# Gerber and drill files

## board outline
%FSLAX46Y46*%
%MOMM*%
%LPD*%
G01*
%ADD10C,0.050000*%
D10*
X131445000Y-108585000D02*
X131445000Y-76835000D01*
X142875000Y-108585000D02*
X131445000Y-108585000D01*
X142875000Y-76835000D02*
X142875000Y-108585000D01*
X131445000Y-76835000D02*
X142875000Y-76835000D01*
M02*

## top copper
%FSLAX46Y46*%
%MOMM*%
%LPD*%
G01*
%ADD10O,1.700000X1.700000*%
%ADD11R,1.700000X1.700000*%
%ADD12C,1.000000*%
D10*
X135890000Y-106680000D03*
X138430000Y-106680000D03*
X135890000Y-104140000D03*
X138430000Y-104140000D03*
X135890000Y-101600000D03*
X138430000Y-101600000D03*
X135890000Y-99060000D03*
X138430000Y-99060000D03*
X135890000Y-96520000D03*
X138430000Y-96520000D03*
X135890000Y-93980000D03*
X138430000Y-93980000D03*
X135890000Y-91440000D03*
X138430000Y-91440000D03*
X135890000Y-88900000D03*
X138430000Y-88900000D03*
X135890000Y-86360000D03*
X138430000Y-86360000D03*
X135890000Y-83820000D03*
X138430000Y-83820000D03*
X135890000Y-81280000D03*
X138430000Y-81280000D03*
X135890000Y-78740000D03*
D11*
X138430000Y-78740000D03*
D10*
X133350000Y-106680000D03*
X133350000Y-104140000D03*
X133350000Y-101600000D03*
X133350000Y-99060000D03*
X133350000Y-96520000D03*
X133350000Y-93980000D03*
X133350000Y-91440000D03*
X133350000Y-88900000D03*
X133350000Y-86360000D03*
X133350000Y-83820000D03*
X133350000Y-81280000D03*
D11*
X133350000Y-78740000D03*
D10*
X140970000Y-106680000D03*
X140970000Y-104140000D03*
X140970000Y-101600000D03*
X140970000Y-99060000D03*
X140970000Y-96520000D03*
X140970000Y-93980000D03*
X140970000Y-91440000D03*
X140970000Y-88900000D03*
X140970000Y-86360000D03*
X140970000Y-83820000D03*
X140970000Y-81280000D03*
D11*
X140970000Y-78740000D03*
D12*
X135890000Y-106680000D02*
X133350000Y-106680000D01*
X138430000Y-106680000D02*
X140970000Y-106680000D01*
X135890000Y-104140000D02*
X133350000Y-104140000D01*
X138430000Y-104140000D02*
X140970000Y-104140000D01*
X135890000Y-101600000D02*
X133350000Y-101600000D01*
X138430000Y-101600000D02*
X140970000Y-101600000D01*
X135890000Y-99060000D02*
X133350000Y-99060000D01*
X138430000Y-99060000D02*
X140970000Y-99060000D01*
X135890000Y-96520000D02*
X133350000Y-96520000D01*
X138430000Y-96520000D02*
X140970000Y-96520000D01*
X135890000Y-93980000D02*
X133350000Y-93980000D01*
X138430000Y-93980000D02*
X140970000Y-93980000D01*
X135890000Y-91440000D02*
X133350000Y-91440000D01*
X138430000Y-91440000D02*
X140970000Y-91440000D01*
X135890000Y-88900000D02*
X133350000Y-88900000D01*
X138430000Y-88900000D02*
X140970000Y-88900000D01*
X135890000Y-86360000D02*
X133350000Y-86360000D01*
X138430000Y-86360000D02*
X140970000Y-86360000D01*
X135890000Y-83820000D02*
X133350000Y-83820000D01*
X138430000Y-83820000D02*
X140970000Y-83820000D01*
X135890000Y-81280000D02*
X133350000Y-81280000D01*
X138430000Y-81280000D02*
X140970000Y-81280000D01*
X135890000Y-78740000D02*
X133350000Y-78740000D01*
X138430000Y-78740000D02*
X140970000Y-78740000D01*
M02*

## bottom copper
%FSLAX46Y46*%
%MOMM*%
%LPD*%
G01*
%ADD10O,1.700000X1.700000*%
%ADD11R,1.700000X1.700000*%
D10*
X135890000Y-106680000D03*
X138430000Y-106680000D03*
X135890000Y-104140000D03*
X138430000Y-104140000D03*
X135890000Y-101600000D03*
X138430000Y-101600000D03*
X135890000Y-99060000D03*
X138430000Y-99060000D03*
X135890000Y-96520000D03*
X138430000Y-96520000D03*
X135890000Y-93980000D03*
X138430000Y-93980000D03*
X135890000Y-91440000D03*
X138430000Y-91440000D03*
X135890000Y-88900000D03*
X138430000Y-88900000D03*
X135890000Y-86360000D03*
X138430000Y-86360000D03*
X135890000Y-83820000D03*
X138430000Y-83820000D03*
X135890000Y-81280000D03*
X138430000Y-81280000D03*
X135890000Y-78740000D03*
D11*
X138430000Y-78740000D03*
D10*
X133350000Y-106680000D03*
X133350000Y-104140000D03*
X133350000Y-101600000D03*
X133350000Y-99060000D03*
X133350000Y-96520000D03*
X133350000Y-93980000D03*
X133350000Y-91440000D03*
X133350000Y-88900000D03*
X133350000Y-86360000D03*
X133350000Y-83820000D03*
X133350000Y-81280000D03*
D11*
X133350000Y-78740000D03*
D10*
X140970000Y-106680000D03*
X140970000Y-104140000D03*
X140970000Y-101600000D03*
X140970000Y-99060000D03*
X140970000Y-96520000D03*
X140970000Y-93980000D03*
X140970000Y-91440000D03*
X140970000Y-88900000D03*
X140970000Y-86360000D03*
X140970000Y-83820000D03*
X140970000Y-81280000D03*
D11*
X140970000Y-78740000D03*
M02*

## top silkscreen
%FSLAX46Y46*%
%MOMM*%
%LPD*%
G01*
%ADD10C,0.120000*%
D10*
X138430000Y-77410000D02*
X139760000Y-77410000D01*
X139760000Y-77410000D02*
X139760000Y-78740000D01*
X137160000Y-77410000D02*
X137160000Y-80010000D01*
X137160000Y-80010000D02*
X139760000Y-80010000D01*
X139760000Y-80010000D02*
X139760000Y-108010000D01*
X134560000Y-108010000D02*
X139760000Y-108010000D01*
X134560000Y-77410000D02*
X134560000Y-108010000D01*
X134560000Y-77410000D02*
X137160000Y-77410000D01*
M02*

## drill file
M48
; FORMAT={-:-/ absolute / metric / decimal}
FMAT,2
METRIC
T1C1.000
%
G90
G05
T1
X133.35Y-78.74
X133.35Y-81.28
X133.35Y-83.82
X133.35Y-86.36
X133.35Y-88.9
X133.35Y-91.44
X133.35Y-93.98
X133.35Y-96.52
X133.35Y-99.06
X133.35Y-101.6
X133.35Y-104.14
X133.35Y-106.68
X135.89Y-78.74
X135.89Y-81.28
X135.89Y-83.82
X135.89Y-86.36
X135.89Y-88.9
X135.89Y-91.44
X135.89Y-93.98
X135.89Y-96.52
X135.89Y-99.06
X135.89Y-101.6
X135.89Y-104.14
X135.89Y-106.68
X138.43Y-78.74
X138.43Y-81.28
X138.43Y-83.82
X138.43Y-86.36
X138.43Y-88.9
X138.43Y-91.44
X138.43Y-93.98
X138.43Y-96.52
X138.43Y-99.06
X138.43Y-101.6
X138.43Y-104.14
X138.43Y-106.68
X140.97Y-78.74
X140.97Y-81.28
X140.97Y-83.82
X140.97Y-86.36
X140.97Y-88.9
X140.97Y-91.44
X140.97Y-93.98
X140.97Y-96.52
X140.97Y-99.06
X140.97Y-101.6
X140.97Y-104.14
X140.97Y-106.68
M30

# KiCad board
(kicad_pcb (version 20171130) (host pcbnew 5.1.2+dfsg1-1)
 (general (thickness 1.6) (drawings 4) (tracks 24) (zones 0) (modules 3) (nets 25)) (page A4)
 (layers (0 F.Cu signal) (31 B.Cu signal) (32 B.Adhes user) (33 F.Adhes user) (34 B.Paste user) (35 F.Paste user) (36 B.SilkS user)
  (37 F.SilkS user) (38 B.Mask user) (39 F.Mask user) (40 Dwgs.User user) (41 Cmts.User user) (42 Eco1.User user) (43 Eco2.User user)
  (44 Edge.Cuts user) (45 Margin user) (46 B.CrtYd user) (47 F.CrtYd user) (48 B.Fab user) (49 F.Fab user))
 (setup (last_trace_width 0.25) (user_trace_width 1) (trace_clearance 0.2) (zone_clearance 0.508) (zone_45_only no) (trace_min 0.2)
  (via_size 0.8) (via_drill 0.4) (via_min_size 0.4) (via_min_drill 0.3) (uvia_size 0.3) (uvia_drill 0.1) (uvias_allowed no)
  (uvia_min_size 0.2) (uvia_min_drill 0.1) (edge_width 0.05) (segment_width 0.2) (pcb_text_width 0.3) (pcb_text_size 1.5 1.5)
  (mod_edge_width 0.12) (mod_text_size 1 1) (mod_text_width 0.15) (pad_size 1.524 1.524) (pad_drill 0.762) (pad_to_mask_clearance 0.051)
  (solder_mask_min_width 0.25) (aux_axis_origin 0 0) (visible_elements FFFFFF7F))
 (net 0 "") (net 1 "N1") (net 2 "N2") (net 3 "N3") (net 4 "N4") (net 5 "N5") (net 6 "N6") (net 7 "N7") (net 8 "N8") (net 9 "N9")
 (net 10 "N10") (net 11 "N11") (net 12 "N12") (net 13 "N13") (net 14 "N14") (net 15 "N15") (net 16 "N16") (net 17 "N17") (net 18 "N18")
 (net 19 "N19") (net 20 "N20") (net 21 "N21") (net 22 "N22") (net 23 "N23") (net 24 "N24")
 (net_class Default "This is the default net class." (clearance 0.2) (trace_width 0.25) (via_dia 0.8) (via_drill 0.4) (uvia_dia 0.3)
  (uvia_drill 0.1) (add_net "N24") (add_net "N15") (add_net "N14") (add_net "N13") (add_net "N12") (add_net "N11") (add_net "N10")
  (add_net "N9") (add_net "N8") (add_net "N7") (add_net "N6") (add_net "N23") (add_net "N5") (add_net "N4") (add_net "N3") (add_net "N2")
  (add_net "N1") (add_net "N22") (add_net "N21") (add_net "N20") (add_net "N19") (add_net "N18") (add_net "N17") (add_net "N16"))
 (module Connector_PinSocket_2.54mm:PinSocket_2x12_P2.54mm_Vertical (layer F.Cu) (at 138.43 78.74)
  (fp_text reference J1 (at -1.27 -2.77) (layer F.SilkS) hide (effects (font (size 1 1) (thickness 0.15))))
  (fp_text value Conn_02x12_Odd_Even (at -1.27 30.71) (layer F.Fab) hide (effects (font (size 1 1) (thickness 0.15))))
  (fp_line (start 0 -1.33) (end 1.33 -1.33) (layer F.SilkS) (width 0.12))
  (fp_line (start 1.33 -1.33) (end 1.33 0) (layer F.SilkS) (width 0.12))
  (fp_line (start -1.27 -1.33) (end -1.27 1.27) (layer F.SilkS) (width 0.12))
  (fp_line (start -1.27 1.27) (end 1.33 1.27) (layer F.SilkS) (width 0.12))
  (fp_line (start 1.33 1.27) (end 1.33 29.27) (layer F.SilkS) (width 0.12))
  (fp_line (start -3.87 29.27) (end 1.33 29.27) (layer F.SilkS) (width 0.12))
  (fp_line (start -3.87 -1.33) (end -3.87 29.27) (layer F.SilkS) (width 0.12))
  (fp_line (start -3.87 -1.33) (end -1.27 -1.33) (layer F.SilkS) (width 0.12))
  (pad 24 thru_hole oval (at -2.54 27.94) (size 1.7 1.7) (drill 1) (layers *.Cu *.Mask) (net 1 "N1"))
  (pad 23 thru_hole oval (at 0 27.94) (size 1.7 1.7) (drill 1) (layers *.Cu *.Mask) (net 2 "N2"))
  (pad 22 thru_hole oval (at -2.54 25.4) (size 1.7 1.7) (drill 1) (layers *.Cu *.Mask) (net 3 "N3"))
  (pad 21 thru_hole oval (at 0 25.4) (size 1.7 1.7) (drill 1) (layers *.Cu *.Mask) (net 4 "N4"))
  (pad 20 thru_hole oval (at -2.54 22.86) (size 1.7 1.7) (drill 1) (layers *.Cu *.Mask) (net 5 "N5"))
  (pad 19 thru_hole oval (at 0 22.86) (size 1.7 1.7) (drill 1) (layers *.Cu *.Mask) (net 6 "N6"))
  (pad 18 thru_hole oval (at -2.54 20.32) (size 1.7 1.7) (drill 1) (layers *.Cu *.Mask) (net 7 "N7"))
  (pad 17 thru_hole oval (at 0 20.32) (size 1.7 1.7) (drill 1) (layers *.Cu *.Mask) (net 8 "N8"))
  (pad 16 thru_hole oval (at -2.54 17.78) (size 1.7 1.7) (drill 1) (layers *.Cu *.Mask) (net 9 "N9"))
  (pad 15 thru_hole oval (at 0 17.78) (size 1.7 1.7) (drill 1) (layers *.Cu *.Mask) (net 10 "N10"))
  (pad 14 thru_hole oval (at -2.54 15.24) (size 1.7 1.7) (drill 1) (layers *.Cu *.Mask) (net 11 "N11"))
  (pad 13 thru_hole oval (at 0 15.24) (size 1.7 1.7) (drill 1) (layers *.Cu *.Mask) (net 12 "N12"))
  (pad 12 thru_hole oval (at -2.54 12.7) (size 1.7 1.7) (drill 1) (layers *.Cu *.Mask) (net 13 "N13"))
  (pad 11 thru_hole oval (at 0 12.7) (size 1.7 1.7) (drill 1) (layers *.Cu *.Mask) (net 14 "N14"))
  (pad 10 thru_hole oval (at -2.54 10.16) (size 1.7 1.7) (drill 1) (layers *.Cu *.Mask) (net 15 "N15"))
  (pad 9 thru_hole oval (at 0 10.16) (size 1.7 1.7) (drill 1) (layers *.Cu *.Mask) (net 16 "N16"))
  (pad 8 thru_hole oval (at -2.54 7.62) (size 1.7 1.7) (drill 1) (layers *.Cu *.Mask) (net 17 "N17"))
  (pad 7 thru_hole oval (at 0 7.62) (size 1.7 1.7) (drill 1) (layers *.Cu *.Mask) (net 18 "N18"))
  (pad 6 thru_hole oval (at -2.54 5.08) (size 1.7 1.7) (drill 1) (layers *.Cu *.Mask) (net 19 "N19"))
  (pad 5 thru_hole oval (at 0 5.08) (size 1.7 1.7) (drill 1) (layers *.Cu *.Mask) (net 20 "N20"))
  (pad 4 thru_hole oval (at -2.54 2.54) (size 1.7 1.7) (drill 1) (layers *.Cu *.Mask) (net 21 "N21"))
  (pad 3 thru_hole oval (at 0 2.54) (size 1.7 1.7) (drill 1) (layers *.Cu *.Mask) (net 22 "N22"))
  (pad 2 thru_hole oval (at -2.54 0) (size 1.7 1.7) (drill 1) (layers *.Cu *.Mask) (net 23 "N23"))
  (pad 1 thru_hole rect (at 0 0) (size 1.7 1.7) (drill 1) (layers *.Cu *.Mask) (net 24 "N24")))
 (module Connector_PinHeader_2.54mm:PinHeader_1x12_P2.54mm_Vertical (layer B.Cu) (at 133.35 78.74 180)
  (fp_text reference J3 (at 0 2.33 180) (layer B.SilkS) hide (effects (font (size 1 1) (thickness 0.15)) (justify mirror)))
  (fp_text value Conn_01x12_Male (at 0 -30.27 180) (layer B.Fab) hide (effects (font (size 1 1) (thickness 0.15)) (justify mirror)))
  (pad 12 thru_hole oval (at 0 -27.94 180) (size 1.7 1.7) (drill 1) (layers *.Cu *.Mask) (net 1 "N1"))
  (pad 11 thru_hole oval (at 0 -25.4 180) (size 1.7 1.7) (drill 1) (layers *.Cu *.Mask) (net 3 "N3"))
  (pad 10 thru_hole oval (at 0 -22.86 180) (size 1.7 1.7) (drill 1) (layers *.Cu *.Mask) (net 5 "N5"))
  (pad 9 thru_hole oval (at 0 -20.32 180) (size 1.7 1.7) (drill 1) (layers *.Cu *.Mask) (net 7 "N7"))
  (pad 8 thru_hole oval (at 0 -17.78 180) (size 1.7 1.7) (drill 1) (layers *.Cu *.Mask) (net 9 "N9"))
  (pad 7 thru_hole oval (at 0 -15.24 180) (size 1.7 1.7) (drill 1) (layers *.Cu *.Mask) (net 11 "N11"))
  (pad 6 thru_hole oval (at 0 -12.7 180) (size 1.7 1.7) (drill 1) (layers *.Cu *.Mask) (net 13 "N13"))
  (pad 5 thru_hole oval (at 0 -10.16 180) (size 1.7 1.7) (drill 1) (layers *.Cu *.Mask) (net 15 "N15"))
  (pad 4 thru_hole oval (at 0 -7.62 180) (size 1.7 1.7) (drill 1) (layers *.Cu *.Mask) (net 17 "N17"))
  (pad 3 thru_hole oval (at 0 -5.08 180) (size 1.7 1.7) (drill 1) (layers *.Cu *.Mask) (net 19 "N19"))
  (pad 2 thru_hole oval (at 0 -2.54 180) (size 1.7 1.7) (drill 1) (layers *.Cu *.Mask) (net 21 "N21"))
  (pad 1 thru_hole rect (at 0 0 180) (size 1.7 1.7) (drill 1) (layers *.Cu *.Mask) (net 23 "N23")))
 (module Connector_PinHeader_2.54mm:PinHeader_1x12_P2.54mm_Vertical (layer B.Cu) (at 140.97 78.74 180)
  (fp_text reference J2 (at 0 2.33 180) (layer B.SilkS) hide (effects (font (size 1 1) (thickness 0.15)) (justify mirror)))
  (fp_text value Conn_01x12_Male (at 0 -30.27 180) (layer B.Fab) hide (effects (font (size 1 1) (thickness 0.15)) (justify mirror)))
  (pad 12 thru_hole oval (at 0 -27.94 180) (size 1.7 1.7) (drill 1) (layers *.Cu *.Mask) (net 2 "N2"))
  (pad 11 thru_hole oval (at 0 -25.4 180) (size 1.7 1.7) (drill 1) (layers *.Cu *.Mask) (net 4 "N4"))
  (pad 10 thru_hole oval (at 0 -22.86 180) (size 1.7 1.7) (drill 1) (layers *.Cu *.Mask) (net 6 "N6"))
  (pad 9 thru_hole oval (at 0 -20.32 180) (size 1.7 1.7) (drill 1) (layers *.Cu *.Mask) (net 8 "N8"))
  (pad 8 thru_hole oval (at 0 -17.78 180) (size 1.7 1.7) (drill 1) (layers *.Cu *.Mask) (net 10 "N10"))
  (pad 7 thru_hole oval (at 0 -15.24 180) (size 1.7 1.7) (drill 1) (layers *.Cu *.Mask) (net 12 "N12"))
  (pad 6 thru_hole oval (at 0 -12.7 180) (size 1.7 1.7) (drill 1) (layers *.Cu *.Mask) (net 14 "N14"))
  (pad 5 thru_hole oval (at 0 -10.16 180) (size 1.7 1.7) (drill 1) (layers *.Cu *.Mask) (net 16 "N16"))
  (pad 4 thru_hole oval (at 0 -7.62 180) (size 1.7 1.7) (drill 1) (layers *.Cu *.Mask) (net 18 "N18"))
  (pad 3 thru_hole oval (at 0 -5.08 180) (size 1.7 1.7) (drill 1) (layers *.Cu *.Mask) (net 20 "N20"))
  (pad 2 thru_hole oval (at 0 -2.54 180) (size 1.7 1.7) (drill 1) (layers *.Cu *.Mask) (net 22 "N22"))
  (pad 1 thru_hole rect (at 0 0 180) (size 1.7 1.7) (drill 1) (layers *.Cu *.Mask) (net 24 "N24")))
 (gr_line (start 131.445 108.585) (end 131.445 76.835) (layer Edge.Cuts) (width 0.05))
 (gr_line (start 142.875 108.585) (end 131.445 108.585) (layer Edge.Cuts) (width 0.05))
 (gr_line (start 142.875 76.835) (end 142.875 108.585) (layer Edge.Cuts) (width 0.05))
 (gr_line (start 131.445 76.835) (end 142.875 76.835) (layer Edge.Cuts) (width 0.05))
 (segment (start 135.89 106.68) (end 133.35 106.68) (width 1) (layer F.Cu) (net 1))
 (segment (start 138.43 106.68) (end 140.97 106.68) (width 1) (layer F.Cu) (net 2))
 (segment (start 135.89 104.14) (end 133.35 104.14) (width 1) (layer F.Cu) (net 3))
 (segment (start 138.43 104.14) (end 140.97 104.14) (width 1) (layer F.Cu) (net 4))
 (segment (start 135.89 101.6) (end 133.35 101.6) (width 1) (layer F.Cu) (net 5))
 (segment (start 138.43 101.6) (end 140.97 101.6) (width 1) (layer F.Cu) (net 6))
 (segment (start 135.89 99.06) (end 133.35 99.06) (width 1) (layer F.Cu) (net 7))
 (segment (start 138.43 99.06) (end 140.97 99.06) (width 1) (layer F.Cu) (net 8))
 (segment (start 135.89 96.52) (end 133.35 96.52) (width 1) (layer F.Cu) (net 9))
 (segment (start 138.43 96.52) (end 140.97 96.52) (width 1) (layer F.Cu) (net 10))
 (segment (start 135.89 93.98) (end 133.35 93.98) (width 1) (layer F.Cu) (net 11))
 (segment (start 138.43 93.98) (end 140.97 93.98) (width 1) (layer F.Cu) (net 12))
 (segment (start 135.89 91.44) (end 133.35 91.44) (width 1) (layer F.Cu) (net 13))
 (segment (start 138.43 91.44) (end 140.97 91.44) (width 1) (layer F.Cu) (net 14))
 (segment (start 135.89 88.9) (end 133.35 88.9) (width 1) (layer F.Cu) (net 15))
 (segment (start 138.43 88.9) (end 140.97 88.9) (width 1) (layer F.Cu) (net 16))
 (segment (start 135.89 86.36) (end 133.35 86.36) (width 1) (layer F.Cu) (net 17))
 (segment (start 138.43 86.36) (end 140.97 86.36) (width 1) (layer F.Cu) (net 18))
 (segment (start 135.89 83.82) (end 133.35 83.82) (width 1) (layer F.Cu) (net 19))
 (segment (start 138.43 83.82) (end 140.97 83.82) (width 1) (layer F.Cu) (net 20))
 (segment (start 135.89 81.28) (end 133.35 81.28) (width 1) (layer F.Cu) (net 21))
 (segment (start 138.43 81.28) (end 140.97 81.28) (width 1) (layer F.Cu) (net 22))
 (segment (start 135.89 78.74) (end 133.35 78.74) (width 1) (layer F.Cu) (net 23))
 (segment (start 138.43 78.74) (end 140.97 78.74) (width 1) (layer F.Cu) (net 24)))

